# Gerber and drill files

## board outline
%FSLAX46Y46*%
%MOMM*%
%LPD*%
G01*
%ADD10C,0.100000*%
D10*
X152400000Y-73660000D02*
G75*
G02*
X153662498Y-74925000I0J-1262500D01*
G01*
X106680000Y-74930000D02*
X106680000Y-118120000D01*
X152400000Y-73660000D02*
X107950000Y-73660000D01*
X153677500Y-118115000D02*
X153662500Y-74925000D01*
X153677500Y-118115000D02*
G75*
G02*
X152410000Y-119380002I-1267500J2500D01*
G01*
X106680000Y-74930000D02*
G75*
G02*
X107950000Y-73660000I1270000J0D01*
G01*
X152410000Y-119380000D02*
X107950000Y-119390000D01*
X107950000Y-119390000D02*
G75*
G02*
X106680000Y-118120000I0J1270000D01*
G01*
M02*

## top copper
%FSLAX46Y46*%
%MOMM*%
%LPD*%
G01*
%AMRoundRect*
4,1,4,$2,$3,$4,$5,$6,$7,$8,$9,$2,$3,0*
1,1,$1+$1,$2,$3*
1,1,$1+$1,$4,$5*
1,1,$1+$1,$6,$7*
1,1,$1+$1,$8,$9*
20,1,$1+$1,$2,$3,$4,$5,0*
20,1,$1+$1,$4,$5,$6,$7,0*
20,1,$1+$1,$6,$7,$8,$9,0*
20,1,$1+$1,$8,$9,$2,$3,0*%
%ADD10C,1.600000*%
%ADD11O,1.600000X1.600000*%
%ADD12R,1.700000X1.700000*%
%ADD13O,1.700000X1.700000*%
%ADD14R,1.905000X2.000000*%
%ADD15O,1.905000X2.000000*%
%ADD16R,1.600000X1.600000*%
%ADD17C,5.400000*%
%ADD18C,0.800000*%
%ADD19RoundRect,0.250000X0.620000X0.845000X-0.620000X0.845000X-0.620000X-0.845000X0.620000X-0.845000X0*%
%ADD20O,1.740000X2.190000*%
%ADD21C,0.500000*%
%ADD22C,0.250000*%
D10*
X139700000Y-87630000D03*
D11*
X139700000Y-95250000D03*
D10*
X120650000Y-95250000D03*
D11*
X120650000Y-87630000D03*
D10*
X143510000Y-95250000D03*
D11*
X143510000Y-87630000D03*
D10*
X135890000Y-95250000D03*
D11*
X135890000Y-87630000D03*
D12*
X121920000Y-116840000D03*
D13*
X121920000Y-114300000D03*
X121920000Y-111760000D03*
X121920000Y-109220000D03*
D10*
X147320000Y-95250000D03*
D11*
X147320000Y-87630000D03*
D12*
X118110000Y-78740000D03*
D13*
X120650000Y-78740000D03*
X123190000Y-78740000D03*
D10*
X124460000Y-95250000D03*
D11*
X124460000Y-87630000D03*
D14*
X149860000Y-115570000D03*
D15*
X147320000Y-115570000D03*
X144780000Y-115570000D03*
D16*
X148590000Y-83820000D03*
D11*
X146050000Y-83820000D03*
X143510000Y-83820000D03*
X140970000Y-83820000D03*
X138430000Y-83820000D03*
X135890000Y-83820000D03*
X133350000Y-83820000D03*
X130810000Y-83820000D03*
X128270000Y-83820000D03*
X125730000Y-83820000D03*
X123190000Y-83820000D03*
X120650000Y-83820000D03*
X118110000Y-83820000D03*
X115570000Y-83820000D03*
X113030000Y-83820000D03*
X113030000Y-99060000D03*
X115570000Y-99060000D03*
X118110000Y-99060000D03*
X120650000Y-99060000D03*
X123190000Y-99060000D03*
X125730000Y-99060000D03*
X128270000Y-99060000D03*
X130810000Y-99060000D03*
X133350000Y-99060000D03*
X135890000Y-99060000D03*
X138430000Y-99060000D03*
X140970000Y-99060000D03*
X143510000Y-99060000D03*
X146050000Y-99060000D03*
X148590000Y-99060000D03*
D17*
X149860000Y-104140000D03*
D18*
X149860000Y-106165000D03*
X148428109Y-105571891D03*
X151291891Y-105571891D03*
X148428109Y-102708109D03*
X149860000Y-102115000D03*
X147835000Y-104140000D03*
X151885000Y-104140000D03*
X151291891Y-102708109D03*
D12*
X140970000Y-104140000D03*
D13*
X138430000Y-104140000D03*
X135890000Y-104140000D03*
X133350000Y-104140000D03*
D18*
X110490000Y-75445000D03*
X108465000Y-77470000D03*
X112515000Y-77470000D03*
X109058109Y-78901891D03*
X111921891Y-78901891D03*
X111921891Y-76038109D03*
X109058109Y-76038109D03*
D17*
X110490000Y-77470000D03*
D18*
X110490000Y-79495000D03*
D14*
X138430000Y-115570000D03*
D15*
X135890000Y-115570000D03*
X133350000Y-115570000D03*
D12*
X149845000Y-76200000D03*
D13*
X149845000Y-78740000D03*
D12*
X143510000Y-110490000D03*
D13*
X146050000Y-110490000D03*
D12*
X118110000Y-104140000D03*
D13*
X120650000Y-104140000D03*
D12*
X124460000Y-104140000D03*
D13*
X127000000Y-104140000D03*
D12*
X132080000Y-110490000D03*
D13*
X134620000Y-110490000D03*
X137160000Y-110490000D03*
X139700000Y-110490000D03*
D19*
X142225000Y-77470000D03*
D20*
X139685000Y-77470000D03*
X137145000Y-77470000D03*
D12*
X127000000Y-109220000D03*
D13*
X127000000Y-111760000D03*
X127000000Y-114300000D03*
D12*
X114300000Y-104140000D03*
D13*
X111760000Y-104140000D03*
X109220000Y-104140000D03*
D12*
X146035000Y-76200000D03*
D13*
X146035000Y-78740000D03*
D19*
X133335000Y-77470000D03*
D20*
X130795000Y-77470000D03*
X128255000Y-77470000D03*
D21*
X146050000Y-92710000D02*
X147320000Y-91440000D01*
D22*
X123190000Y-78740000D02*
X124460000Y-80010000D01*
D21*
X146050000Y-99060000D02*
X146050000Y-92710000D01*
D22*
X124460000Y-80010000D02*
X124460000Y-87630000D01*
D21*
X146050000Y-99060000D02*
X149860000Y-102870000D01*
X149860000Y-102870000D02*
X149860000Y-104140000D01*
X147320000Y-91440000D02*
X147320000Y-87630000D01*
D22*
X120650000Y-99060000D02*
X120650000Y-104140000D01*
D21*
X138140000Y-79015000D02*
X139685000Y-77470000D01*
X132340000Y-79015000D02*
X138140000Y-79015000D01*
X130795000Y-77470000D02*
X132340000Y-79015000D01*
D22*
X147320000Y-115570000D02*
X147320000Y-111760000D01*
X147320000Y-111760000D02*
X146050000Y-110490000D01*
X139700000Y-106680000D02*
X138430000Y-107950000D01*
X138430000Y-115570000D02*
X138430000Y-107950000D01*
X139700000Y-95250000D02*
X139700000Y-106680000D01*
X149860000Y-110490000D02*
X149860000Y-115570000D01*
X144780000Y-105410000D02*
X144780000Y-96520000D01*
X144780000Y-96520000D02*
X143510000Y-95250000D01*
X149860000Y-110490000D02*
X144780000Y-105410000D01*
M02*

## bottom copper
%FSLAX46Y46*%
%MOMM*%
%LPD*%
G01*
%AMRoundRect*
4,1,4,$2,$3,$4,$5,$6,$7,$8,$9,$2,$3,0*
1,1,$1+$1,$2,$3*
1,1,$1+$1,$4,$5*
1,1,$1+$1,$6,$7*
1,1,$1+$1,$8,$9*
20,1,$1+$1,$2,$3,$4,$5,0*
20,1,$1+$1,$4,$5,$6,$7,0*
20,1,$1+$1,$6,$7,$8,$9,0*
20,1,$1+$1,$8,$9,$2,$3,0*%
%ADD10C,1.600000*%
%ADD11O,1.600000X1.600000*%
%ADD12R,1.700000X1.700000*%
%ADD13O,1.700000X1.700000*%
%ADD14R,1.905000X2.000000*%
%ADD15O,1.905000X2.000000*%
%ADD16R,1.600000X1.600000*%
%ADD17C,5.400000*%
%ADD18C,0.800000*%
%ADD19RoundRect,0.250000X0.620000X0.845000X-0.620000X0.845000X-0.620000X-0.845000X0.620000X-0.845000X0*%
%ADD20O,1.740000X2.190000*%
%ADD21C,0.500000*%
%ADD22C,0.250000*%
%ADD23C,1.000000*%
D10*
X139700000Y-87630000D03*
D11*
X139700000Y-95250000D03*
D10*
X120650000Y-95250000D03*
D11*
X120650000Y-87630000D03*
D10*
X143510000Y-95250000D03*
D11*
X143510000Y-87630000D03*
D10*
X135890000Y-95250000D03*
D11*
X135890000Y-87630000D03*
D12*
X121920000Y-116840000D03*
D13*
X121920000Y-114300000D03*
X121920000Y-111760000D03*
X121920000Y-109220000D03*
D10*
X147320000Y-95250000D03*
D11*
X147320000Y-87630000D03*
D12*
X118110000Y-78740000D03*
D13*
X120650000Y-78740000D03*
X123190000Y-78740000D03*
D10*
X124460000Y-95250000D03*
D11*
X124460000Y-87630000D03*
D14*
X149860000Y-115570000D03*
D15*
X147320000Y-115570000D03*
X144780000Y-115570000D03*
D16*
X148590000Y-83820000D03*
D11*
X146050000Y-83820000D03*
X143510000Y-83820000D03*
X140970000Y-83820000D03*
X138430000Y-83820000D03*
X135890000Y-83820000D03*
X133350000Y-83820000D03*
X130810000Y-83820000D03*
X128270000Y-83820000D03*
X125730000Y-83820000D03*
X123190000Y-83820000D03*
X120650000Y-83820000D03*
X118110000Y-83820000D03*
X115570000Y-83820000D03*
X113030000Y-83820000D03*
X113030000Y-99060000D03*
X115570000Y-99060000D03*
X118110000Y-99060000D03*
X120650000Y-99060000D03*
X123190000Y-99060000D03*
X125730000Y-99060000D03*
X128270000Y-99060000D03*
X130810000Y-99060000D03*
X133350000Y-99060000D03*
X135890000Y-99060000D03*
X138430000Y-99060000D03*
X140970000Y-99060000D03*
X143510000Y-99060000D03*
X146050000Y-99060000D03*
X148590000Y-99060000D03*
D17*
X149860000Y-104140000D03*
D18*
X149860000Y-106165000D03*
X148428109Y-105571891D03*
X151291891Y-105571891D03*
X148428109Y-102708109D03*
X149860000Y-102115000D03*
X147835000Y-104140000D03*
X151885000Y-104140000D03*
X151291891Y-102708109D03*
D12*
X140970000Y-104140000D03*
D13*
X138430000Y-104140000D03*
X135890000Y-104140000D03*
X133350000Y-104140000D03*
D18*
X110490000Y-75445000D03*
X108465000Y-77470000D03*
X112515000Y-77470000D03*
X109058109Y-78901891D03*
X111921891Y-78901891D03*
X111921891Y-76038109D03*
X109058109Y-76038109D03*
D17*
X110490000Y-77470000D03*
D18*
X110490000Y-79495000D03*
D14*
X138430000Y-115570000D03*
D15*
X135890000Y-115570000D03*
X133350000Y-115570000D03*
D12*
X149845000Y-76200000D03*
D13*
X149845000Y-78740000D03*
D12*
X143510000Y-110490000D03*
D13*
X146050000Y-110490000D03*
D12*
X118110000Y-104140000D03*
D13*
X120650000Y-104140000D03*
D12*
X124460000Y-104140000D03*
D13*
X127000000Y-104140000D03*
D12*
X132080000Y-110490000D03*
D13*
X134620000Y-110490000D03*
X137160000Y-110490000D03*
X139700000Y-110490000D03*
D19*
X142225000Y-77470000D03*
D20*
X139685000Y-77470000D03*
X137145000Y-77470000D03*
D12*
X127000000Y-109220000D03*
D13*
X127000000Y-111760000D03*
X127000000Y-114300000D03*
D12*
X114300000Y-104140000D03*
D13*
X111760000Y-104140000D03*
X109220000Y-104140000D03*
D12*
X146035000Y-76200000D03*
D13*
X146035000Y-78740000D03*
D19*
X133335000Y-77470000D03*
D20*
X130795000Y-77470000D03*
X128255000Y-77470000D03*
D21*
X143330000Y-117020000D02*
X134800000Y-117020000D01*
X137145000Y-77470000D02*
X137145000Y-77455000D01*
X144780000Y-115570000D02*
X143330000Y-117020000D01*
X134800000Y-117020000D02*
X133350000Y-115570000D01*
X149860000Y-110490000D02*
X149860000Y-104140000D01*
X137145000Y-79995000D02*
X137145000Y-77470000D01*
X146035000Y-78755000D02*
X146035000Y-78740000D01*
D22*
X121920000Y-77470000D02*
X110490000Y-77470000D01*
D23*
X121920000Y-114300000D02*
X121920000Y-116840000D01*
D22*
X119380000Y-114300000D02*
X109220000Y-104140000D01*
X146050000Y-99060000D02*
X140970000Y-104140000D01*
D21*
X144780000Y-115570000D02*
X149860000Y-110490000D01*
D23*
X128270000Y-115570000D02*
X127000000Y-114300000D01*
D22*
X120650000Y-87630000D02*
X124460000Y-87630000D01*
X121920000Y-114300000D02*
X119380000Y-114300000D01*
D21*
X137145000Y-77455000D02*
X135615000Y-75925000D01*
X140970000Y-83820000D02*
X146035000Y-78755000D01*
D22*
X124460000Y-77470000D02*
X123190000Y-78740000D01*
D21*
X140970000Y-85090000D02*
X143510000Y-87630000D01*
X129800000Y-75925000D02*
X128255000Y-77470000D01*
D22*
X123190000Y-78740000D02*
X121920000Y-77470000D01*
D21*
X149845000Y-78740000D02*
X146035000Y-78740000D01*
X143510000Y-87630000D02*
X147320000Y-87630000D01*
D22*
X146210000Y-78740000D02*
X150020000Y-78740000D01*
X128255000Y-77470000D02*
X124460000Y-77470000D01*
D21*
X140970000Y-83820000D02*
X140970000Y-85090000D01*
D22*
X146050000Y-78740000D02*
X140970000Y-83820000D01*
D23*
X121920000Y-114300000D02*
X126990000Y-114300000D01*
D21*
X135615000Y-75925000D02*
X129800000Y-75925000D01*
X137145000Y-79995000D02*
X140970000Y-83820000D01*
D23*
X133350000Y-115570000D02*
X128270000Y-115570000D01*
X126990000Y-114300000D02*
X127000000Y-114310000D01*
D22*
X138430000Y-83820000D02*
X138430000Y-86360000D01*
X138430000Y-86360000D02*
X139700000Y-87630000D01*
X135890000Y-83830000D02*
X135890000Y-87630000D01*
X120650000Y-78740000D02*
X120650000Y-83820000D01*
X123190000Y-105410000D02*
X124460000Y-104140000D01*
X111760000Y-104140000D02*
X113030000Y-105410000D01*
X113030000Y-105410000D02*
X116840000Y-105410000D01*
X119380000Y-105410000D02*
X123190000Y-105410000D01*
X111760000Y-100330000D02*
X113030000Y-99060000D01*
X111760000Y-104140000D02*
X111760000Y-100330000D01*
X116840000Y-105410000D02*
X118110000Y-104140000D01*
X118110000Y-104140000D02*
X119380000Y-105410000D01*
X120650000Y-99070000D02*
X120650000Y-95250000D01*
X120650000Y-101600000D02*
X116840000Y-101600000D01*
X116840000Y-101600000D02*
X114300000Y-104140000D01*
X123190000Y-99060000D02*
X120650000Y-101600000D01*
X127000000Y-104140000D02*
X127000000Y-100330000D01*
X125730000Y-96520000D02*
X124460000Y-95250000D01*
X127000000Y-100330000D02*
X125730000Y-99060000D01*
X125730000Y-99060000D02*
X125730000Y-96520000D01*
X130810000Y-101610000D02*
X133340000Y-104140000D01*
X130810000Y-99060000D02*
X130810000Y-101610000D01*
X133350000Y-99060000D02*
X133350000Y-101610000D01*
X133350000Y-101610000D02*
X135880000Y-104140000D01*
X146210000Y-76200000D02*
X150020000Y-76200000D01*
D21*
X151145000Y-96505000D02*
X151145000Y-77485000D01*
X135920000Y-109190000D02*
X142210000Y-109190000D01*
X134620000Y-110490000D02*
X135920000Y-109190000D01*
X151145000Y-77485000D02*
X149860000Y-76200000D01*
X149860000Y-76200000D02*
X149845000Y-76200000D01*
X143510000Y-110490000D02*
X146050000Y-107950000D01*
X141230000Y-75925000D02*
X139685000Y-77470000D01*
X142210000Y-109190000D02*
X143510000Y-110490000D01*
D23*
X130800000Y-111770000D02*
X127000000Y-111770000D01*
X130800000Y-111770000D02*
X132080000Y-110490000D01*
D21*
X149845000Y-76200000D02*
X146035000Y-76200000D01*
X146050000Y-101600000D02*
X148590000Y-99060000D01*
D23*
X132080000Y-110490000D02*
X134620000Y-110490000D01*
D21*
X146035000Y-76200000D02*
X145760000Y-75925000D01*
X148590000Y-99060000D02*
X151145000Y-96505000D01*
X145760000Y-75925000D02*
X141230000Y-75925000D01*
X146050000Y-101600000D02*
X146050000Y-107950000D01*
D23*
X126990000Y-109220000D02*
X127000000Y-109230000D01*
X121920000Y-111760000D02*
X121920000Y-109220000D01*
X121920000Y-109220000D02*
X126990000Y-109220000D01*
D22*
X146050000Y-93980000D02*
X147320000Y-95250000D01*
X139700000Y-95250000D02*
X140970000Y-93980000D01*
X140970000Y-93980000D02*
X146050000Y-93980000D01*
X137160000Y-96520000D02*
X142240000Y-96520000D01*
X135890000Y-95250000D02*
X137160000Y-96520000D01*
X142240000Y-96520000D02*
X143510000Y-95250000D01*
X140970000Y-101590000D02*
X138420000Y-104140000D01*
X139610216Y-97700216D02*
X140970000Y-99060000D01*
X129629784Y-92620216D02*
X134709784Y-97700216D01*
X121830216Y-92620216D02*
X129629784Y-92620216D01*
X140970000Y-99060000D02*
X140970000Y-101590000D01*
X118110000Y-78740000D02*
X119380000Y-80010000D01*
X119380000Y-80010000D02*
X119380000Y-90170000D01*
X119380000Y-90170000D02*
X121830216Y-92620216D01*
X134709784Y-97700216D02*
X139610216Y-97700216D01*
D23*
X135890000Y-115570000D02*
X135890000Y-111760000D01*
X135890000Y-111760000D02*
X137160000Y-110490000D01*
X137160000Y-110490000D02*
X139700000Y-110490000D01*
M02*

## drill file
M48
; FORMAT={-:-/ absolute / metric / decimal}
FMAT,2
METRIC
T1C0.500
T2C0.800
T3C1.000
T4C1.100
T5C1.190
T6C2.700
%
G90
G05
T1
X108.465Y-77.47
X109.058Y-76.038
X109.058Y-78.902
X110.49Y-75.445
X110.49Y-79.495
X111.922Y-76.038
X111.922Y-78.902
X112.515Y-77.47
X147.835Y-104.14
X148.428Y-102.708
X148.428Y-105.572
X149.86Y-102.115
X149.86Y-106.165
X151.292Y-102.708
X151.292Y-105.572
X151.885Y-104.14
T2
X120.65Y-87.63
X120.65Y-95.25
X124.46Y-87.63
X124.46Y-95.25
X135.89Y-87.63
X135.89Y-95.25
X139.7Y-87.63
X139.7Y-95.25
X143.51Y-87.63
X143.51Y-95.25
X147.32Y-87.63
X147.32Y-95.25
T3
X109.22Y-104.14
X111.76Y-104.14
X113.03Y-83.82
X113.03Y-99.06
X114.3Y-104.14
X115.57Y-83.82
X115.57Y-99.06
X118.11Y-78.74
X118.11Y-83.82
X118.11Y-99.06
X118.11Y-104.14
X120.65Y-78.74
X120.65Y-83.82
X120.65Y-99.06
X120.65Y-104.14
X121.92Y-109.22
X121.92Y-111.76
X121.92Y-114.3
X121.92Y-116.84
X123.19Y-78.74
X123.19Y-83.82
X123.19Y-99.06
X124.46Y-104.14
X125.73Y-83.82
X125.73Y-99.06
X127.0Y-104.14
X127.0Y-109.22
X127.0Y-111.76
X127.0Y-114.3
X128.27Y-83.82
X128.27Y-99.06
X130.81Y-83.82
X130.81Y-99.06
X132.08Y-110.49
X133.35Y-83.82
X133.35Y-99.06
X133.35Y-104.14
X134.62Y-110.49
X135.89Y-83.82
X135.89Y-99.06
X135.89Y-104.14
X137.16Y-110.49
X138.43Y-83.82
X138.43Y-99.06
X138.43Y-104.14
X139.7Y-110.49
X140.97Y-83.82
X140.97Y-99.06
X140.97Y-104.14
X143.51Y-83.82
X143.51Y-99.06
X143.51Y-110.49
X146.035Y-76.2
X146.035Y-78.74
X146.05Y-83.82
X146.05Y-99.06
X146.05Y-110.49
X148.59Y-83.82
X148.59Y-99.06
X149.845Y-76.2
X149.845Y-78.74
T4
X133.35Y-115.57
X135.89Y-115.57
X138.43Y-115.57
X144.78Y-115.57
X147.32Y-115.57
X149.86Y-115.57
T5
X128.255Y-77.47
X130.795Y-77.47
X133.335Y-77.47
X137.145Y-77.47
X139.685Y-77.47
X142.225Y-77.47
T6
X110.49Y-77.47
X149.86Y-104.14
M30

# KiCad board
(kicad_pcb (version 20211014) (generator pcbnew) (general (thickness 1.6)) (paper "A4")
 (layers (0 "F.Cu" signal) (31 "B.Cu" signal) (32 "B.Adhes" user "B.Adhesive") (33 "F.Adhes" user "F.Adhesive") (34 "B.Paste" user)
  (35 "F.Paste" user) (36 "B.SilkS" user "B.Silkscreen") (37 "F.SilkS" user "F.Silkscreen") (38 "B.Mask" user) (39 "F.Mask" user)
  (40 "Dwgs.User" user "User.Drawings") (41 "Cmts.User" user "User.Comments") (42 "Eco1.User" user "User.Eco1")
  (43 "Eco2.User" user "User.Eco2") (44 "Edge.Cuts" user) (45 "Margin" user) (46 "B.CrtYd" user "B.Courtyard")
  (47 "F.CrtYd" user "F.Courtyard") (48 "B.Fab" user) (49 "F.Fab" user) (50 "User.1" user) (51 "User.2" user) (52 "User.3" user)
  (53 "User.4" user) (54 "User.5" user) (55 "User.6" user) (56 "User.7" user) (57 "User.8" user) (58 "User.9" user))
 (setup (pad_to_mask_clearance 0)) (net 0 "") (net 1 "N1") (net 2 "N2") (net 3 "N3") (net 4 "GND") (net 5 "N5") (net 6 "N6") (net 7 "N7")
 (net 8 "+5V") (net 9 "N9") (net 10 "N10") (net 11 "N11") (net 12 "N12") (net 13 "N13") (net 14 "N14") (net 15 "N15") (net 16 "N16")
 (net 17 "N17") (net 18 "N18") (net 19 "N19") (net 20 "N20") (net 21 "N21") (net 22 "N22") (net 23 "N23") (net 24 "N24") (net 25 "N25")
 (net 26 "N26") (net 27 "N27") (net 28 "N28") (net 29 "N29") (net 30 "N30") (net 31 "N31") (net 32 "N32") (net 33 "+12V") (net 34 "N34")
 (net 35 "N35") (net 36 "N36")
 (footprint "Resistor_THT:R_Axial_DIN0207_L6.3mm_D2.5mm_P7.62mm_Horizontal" (layer "F.Cu") (at 139.7 87.63 -90)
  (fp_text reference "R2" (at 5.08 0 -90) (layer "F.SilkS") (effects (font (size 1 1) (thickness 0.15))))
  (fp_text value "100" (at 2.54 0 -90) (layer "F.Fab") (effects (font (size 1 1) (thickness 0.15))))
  (pad "1" thru_hole circle (at 0 0 270) (size 1.6 1.6) (drill 0.8) (layers *.Cu *.Mask) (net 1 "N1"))
  (pad "2" thru_hole oval (at 7.62 0 270) (size 1.6 1.6) (drill 0.8) (layers *.Cu *.Mask) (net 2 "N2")))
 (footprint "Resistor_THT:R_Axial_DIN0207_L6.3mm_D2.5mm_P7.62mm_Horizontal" (layer "F.Cu") (at 120.65 95.25 90)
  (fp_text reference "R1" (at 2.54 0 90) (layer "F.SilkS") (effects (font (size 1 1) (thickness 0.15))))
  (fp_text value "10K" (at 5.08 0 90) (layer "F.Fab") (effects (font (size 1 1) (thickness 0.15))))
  (pad "1" thru_hole circle (at 0 0 90) (size 1.6 1.6) (drill 0.8) (layers *.Cu *.Mask) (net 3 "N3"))
  (pad "2" thru_hole oval (at 7.62 0 90) (size 1.6 1.6) (drill 0.8) (layers *.Cu *.Mask) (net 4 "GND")))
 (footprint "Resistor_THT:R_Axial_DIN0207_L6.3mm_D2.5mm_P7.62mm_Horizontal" (layer "F.Cu") (at 143.51 95.25 90)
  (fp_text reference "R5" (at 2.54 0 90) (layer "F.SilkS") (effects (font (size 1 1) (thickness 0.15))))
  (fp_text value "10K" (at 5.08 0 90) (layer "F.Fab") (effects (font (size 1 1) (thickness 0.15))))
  (pad "1" thru_hole circle (at 0 0 90) (size 1.6 1.6) (drill 0.8) (layers *.Cu *.Mask) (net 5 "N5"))
  (pad "2" thru_hole oval (at 7.62 0 90) (size 1.6 1.6) (drill 0.8) (layers *.Cu *.Mask) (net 4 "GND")))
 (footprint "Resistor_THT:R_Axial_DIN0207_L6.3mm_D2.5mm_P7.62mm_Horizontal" (layer "F.Cu") (at 135.89 95.25 90)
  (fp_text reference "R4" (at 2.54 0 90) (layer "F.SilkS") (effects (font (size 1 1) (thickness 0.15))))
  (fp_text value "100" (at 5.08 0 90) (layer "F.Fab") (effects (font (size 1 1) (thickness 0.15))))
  (pad "1" thru_hole circle (at 0 0 90) (size 1.6 1.6) (drill 0.8) (layers *.Cu *.Mask) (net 5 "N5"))
  (pad "2" thru_hole oval (at 7.62 0 90) (size 1.6 1.6) (drill 0.8) (layers *.Cu *.Mask) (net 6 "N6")))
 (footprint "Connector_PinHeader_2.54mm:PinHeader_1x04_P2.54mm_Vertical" (layer "F.Cu") (at 121.92 116.84 180)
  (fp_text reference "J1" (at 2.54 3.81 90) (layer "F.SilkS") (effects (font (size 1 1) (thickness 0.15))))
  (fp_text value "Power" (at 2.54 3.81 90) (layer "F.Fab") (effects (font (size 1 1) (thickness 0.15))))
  (pad "1" thru_hole rect (at 0 0 180) (size 1.7 1.7) (drill 1) (layers *.Cu *.Mask) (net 4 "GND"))
  (pad "2" thru_hole oval (at 0 2.54 180) (size 1.7 1.7) (drill 1) (layers *.Cu *.Mask) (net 4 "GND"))
  (pad "3" thru_hole oval (at 0 5.08 180) (size 1.7 1.7) (drill 1) (layers *.Cu *.Mask) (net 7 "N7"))
  (pad "4" thru_hole oval (at 0 7.62 180) (size 1.7 1.7) (drill 1) (layers *.Cu *.Mask) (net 7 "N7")))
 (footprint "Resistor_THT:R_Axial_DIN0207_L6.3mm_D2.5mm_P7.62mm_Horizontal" (layer "F.Cu") (at 147.32 95.25 90)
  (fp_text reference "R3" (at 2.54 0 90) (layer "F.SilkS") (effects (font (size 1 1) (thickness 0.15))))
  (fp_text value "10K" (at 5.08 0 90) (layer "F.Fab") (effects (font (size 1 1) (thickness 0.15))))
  (pad "1" thru_hole circle (at 0 0 90) (size 1.6 1.6) (drill 0.8) (layers *.Cu *.Mask) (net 2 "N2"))
  (pad "2" thru_hole oval (at 7.62 0 90) (size 1.6 1.6) (drill 0.8) (layers *.Cu *.Mask) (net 4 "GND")))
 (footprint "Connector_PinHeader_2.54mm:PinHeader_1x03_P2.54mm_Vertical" (layer "F.Cu") (at 118.11 78.74 90)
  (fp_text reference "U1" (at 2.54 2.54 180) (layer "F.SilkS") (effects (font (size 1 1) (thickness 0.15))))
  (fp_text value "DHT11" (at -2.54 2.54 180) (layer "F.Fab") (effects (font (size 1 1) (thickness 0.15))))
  (pad "1" thru_hole rect (at 0 0 90) (size 1.7 1.7) (drill 1) (layers *.Cu *.Mask) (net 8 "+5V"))
  (pad "2" thru_hole oval (at 0 2.54 90) (size 1.7 1.7) (drill 1) (layers *.Cu *.Mask) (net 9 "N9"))
  (pad "3" thru_hole oval (at 0 5.08 90) (size 1.7 1.7) (drill 1) (layers *.Cu *.Mask) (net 4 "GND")))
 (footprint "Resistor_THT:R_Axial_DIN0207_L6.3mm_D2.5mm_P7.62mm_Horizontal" (layer "F.Cu") (at 124.46 95.25 90)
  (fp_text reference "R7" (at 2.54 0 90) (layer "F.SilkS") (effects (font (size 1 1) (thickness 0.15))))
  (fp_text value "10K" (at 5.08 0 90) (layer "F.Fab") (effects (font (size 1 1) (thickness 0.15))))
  (pad "1" thru_hole circle (at 0 0 90) (size 1.6 1.6) (drill 0.8) (layers *.Cu *.Mask) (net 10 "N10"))
  (pad "2" thru_hole oval (at 7.62 0 90) (size 1.6 1.6) (drill 0.8) (layers *.Cu *.Mask) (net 4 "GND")))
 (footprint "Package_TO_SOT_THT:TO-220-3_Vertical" (layer "F.Cu") (at 149.86 115.57 180)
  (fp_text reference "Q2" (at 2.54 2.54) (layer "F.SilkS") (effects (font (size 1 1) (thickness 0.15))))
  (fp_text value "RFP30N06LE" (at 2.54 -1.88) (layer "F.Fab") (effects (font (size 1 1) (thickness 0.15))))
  (pad "1" thru_hole rect (at 0 0 180) (size 1.905 2) (drill 1.1) (layers *.Cu *.Mask) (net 5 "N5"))
  (pad "2" thru_hole oval (at 2.54 0 180) (size 1.905 2) (drill 1.1) (layers *.Cu *.Mask) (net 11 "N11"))
  (pad "3" thru_hole oval (at 5.08 0 180) (size 1.905 2) (drill 1.1) (layers *.Cu *.Mask) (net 4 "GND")))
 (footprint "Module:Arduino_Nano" (layer "F.Cu") (at 148.59 83.82 -90)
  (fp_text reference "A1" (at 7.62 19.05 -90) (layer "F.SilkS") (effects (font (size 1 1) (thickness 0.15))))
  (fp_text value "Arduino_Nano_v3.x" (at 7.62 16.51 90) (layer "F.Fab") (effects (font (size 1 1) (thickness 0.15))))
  (pad "1" thru_hole rect (at 0 0 270) (size 1.6 1.6) (drill 1) (layers *.Cu *.Mask) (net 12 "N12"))
  (pad "2" thru_hole oval (at 0 2.54 270) (size 1.6 1.6) (drill 1) (layers *.Cu *.Mask) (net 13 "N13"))
  (pad "3" thru_hole oval (at 0 5.08 270) (size 1.6 1.6) (drill 1) (layers *.Cu *.Mask) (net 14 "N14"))
  (pad "4" thru_hole oval (at 0 7.62 270) (size 1.6 1.6) (drill 1) (layers *.Cu *.Mask) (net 4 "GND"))
  (pad "5" thru_hole oval (at 0 10.16 270) (size 1.6 1.6) (drill 1) (layers *.Cu *.Mask) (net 1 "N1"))
  (pad "6" thru_hole oval (at 0 12.7 270) (size 1.6 1.6) (drill 1) (layers *.Cu *.Mask) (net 6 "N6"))
  (pad "7" thru_hole oval (at 0 15.24 270) (size 1.6 1.6) (drill 1) (layers *.Cu *.Mask) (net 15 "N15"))
  (pad "8" thru_hole oval (at 0 17.78 270) (size 1.6 1.6) (drill 1) (layers *.Cu *.Mask) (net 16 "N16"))
  (pad "9" thru_hole oval (at 0 20.32 270) (size 1.6 1.6) (drill 1) (layers *.Cu *.Mask) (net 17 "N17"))
  (pad "10" thru_hole oval (at 0 22.86 270) (size 1.6 1.6) (drill 1) (layers *.Cu *.Mask) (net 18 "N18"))
  (pad "11" thru_hole oval (at 0 25.4 270) (size 1.6 1.6) (drill 1) (layers *.Cu *.Mask) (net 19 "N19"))
  (pad "12" thru_hole oval (at 0 27.94 270) (size 1.6 1.6) (drill 1) (layers *.Cu *.Mask) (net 9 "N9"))
  (pad "13" thru_hole oval (at 0 30.48 270) (size 1.6 1.6) (drill 1) (layers *.Cu *.Mask) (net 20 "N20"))
  (pad "14" thru_hole oval (at 0 33.02 270) (size 1.6 1.6) (drill 1) (layers *.Cu *.Mask) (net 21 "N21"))
  (pad "15" thru_hole oval (at 0 35.56 270) (size 1.6 1.6) (drill 1) (layers *.Cu *.Mask) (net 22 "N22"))
  (pad "16" thru_hole oval (at 15.24 35.56 270) (size 1.6 1.6) (drill 1) (layers *.Cu *.Mask) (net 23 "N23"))
  (pad "17" thru_hole oval (at 15.24 33.02 270) (size 1.6 1.6) (drill 1) (layers *.Cu *.Mask) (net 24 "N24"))
  (pad "18" thru_hole oval (at 15.24 30.48 270) (size 1.6 1.6) (drill 1) (layers *.Cu *.Mask) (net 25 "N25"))
  (pad "19" thru_hole oval (at 15.24 27.94 270) (size 1.6 1.6) (drill 1) (layers *.Cu *.Mask) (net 3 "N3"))
  (pad "20" thru_hole oval (at 15.24 25.4 270) (size 1.6 1.6) (drill 1) (layers *.Cu *.Mask) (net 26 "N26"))
  (pad "21" thru_hole oval (at 15.24 22.86 270) (size 1.6 1.6) (drill 1) (layers *.Cu *.Mask) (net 10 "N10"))
  (pad "22" thru_hole oval (at 15.24 20.32 270) (size 1.6 1.6) (drill 1) (layers *.Cu *.Mask) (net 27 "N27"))
  (pad "23" thru_hole oval (at 15.24 17.78 270) (size 1.6 1.6) (drill 1) (layers *.Cu *.Mask) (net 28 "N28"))
  (pad "24" thru_hole oval (at 15.24 15.24 270) (size 1.6 1.6) (drill 1) (layers *.Cu *.Mask) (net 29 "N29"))
  (pad "25" thru_hole oval (at 15.24 12.7 270) (size 1.6 1.6) (drill 1) (layers *.Cu *.Mask) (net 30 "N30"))
  (pad "26" thru_hole oval (at 15.24 10.16 270) (size 1.6 1.6) (drill 1) (layers *.Cu *.Mask) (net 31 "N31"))
  (pad "27" thru_hole oval (at 15.24 7.62 270) (size 1.6 1.6) (drill 1) (layers *.Cu *.Mask) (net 8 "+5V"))
  (pad "28" thru_hole oval (at 15.24 5.08 270) (size 1.6 1.6) (drill 1) (layers *.Cu *.Mask) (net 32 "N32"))
  (pad "29" thru_hole oval (at 15.24 2.54 270) (size 1.6 1.6) (drill 1) (layers *.Cu *.Mask) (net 4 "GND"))
  (pad "30" thru_hole oval (at 15.24 0 270) (size 1.6 1.6) (drill 1) (layers *.Cu *.Mask) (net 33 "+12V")))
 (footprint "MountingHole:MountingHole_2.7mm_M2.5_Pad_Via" (layer "F.Cu") (at 149.86 104.14)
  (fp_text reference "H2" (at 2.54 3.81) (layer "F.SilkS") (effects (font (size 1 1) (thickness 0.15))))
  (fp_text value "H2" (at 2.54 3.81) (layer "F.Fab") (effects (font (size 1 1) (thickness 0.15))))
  (pad "1" thru_hole circle (at 0 0) (size 5.4 5.4) (drill 2.7) (layers *.Cu *.Mask) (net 4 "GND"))
  (pad "1" thru_hole circle (at 0 2.025) (size 0.8 0.8) (drill 0.5) (layers *.Cu *.Mask) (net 4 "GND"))
  (pad "1" thru_hole circle (at -1.431891 1.431891) (size 0.8 0.8) (drill 0.5) (layers *.Cu *.Mask) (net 4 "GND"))
  (pad "1" thru_hole circle (at 1.431891 1.431891) (size 0.8 0.8) (drill 0.5) (layers *.Cu *.Mask) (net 4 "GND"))
  (pad "1" thru_hole circle (at -1.431891 -1.431891) (size 0.8 0.8) (drill 0.5) (layers *.Cu *.Mask) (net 4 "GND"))
  (pad "1" thru_hole circle (at 0 -2.025) (size 0.8 0.8) (drill 0.5) (layers *.Cu *.Mask) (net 4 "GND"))
  (pad "1" thru_hole circle (at -2.025 0) (size 0.8 0.8) (drill 0.5) (layers *.Cu *.Mask) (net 4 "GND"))
  (pad "1" thru_hole circle (at 2.025 0) (size 0.8 0.8) (drill 0.5) (layers *.Cu *.Mask) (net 4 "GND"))
  (pad "1" thru_hole circle (at 1.431891 -1.431891) (size 0.8 0.8) (drill 0.5) (layers *.Cu *.Mask) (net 4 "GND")))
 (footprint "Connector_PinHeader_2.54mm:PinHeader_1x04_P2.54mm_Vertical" (layer "F.Cu") (at 140.97 104.14 -90)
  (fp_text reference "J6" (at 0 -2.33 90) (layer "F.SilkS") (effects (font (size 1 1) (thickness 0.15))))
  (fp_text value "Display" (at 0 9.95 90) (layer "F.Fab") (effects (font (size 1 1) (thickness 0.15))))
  (pad "1" thru_hole rect (at 0 0 270) (size 1.7 1.7) (drill 1) (layers *.Cu *.Mask) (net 4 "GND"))
  (pad "2" thru_hole oval (at 0 2.54 270) (size 1.7 1.7) (drill 1) (layers *.Cu *.Mask) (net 8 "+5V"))
  (pad "3" thru_hole oval (at 0 5.08 270) (size 1.7 1.7) (drill 1) (layers *.Cu *.Mask) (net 29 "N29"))
  (pad "4" thru_hole oval (at 0 7.62 270) (size 1.7 1.7) (drill 1) (layers *.Cu *.Mask) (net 28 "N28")))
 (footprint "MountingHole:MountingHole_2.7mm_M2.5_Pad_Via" (layer "F.Cu") (at 110.49 77.47)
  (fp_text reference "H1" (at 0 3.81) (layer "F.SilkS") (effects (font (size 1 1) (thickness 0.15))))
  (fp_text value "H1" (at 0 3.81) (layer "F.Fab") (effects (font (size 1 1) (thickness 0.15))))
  (pad "1" thru_hole circle (at 0 -2.025) (size 0.8 0.8) (drill 0.5) (layers *.Cu *.Mask) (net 4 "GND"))
  (pad "1" thru_hole circle (at -2.025 0) (size 0.8 0.8) (drill 0.5) (layers *.Cu *.Mask) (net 4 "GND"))
  (pad "1" thru_hole circle (at 2.025 0) (size 0.8 0.8) (drill 0.5) (layers *.Cu *.Mask) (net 4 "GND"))
  (pad "1" thru_hole circle (at -1.431891 1.431891) (size 0.8 0.8) (drill 0.5) (layers *.Cu *.Mask) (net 4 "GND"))
  (pad "1" thru_hole circle (at 1.431891 1.431891) (size 0.8 0.8) (drill 0.5) (layers *.Cu *.Mask) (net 4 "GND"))
  (pad "1" thru_hole circle (at 1.431891 -1.431891) (size 0.8 0.8) (drill 0.5) (layers *.Cu *.Mask) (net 4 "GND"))
  (pad "1" thru_hole circle (at -1.431891 -1.431891) (size 0.8 0.8) (drill 0.5) (layers *.Cu *.Mask) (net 4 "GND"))
  (pad "1" thru_hole circle (at 0 0) (size 5.4 5.4) (drill 2.7) (layers *.Cu *.Mask) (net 4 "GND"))
  (pad "1" thru_hole circle (at 0 2.025) (size 0.8 0.8) (drill 0.5) (layers *.Cu *.Mask) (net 4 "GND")))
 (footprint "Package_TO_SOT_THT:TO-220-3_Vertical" (layer "F.Cu") (at 138.43 115.57 180)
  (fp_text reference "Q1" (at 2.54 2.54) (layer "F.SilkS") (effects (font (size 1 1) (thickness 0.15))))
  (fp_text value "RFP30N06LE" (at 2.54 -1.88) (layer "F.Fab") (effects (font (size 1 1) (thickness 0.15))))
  (pad "1" thru_hole rect (at 0 0 180) (size 1.905 2) (drill 1.1) (layers *.Cu *.Mask) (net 2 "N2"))
  (pad "2" thru_hole oval (at 2.54 0 180) (size 1.905 2) (drill 1.1) (layers *.Cu *.Mask) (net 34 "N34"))
  (pad "3" thru_hole oval (at 5.08 0 180) (size 1.905 2) (drill 1.1) (layers *.Cu *.Mask) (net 4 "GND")))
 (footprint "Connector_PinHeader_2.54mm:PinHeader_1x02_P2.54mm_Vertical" (layer "B.Cu") (at 149.845 76.2 180)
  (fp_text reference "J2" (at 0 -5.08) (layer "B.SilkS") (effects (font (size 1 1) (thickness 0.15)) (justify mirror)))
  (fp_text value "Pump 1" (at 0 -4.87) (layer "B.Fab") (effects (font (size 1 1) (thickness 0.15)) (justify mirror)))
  (pad "1" thru_hole rect (at 0 0 180) (size 1.7 1.7) (drill 1) (layers *.Cu *.Mask) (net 33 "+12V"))
  (pad "2" thru_hole oval (at 0 -2.54 180) (size 1.7 1.7) (drill 1) (layers *.Cu *.Mask) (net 4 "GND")))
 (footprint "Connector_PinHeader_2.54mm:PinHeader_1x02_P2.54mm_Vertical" (layer "B.Cu") (at 143.51 110.49 -90)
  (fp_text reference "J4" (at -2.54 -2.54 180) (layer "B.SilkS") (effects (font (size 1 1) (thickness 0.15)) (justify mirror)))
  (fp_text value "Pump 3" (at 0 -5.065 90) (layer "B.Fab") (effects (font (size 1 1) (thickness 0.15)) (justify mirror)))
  (pad "1" thru_hole rect (at 0 0 270) (size 1.7 1.7) (drill 1) (layers *.Cu *.Mask) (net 33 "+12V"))
  (pad "2" thru_hole oval (at 0 -2.54 270) (size 1.7 1.7) (drill 1) (layers *.Cu *.Mask) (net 11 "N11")))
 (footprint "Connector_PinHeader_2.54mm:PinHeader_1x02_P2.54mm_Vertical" (layer "B.Cu") (at 118.11 104.14 -90)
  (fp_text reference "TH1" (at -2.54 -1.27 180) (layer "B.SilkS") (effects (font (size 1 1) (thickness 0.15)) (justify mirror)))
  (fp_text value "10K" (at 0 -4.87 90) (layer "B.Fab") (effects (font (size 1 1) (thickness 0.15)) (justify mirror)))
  (pad "1" thru_hole rect (at 0 0 270) (size 1.7 1.7) (drill 1) (layers *.Cu *.Mask) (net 23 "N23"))
  (pad "2" thru_hole oval (at 0 -2.54 270) (size 1.7 1.7) (drill 1) (layers *.Cu *.Mask) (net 3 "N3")))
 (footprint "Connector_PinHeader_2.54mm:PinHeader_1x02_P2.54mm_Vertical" (layer "B.Cu") (at 124.46 104.14 -90)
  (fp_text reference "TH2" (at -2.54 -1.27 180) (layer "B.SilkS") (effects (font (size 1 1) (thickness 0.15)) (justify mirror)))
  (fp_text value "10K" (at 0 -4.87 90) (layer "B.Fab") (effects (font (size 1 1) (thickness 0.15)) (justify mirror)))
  (pad "1" thru_hole rect (at 0 0 270) (size 1.7 1.7) (drill 1) (layers *.Cu *.Mask) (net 23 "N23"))
  (pad "2" thru_hole oval (at 0 -2.54 270) (size 1.7 1.7) (drill 1) (layers *.Cu *.Mask) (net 10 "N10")))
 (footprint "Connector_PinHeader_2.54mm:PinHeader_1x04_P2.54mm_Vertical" (layer "B.Cu") (at 132.08 110.49 -90)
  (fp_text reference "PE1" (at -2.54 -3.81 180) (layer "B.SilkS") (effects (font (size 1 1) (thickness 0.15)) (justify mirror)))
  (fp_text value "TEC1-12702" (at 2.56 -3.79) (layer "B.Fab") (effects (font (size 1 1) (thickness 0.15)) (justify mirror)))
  (pad "1" thru_hole rect (at 0 0 270) (size 1.7 1.7) (drill 1) (layers *.Cu *.Mask) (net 33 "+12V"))
  (pad "2" thru_hole oval (at 0 -2.54 270) (size 1.7 1.7) (drill 1) (layers *.Cu *.Mask) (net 33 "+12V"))
  (pad "3" thru_hole oval (at 0 -5.08 270) (size 1.7 1.7) (drill 1) (layers *.Cu *.Mask) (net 34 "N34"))
  (pad "4" thru_hole oval (at 0 -7.62 270) (size 1.7 1.7) (drill 1) (layers *.Cu *.Mask) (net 34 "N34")))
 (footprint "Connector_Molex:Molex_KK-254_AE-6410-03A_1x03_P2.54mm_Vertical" (layer "B.Cu") (at 142.225 77.47 180)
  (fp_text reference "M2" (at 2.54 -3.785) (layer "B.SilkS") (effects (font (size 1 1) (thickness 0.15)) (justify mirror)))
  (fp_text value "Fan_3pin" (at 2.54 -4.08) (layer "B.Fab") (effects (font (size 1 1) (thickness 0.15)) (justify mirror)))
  (pad "1" thru_hole roundrect (at 0 0 180) (size 1.74 2.19) (drill 1.19) (layers *.Cu *.Mask) (roundrect_rratio 0.1436781609)
   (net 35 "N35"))
  (pad "2" thru_hole oval (at 2.54 0 180) (size 1.74 2.19) (drill 1.19) (layers *.Cu *.Mask) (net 33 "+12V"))
  (pad "3" thru_hole oval (at 5.08 0 180) (size 1.74 2.19) (drill 1.19) (layers *.Cu *.Mask) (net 4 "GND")))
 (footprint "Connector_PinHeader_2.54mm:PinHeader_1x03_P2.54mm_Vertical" (layer "B.Cu") (at 127 109.22 180)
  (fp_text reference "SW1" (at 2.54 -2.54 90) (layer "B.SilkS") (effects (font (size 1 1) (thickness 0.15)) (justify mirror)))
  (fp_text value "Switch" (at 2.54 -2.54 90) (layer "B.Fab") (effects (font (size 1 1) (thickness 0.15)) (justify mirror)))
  (pad "1" thru_hole rect (at 0 0 180) (size 1.7 1.7) (drill 1) (layers *.Cu *.Mask) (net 7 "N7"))
  (pad "2" thru_hole oval (at 0 -2.54 180) (size 1.7 1.7) (drill 1) (layers *.Cu *.Mask) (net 33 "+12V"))
  (pad "3" thru_hole oval (at 0 -5.08 180) (size 1.7 1.7) (drill 1) (layers *.Cu *.Mask) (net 4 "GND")))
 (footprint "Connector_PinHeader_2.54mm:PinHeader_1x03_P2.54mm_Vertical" (layer "B.Cu") (at 114.3 104.14 90)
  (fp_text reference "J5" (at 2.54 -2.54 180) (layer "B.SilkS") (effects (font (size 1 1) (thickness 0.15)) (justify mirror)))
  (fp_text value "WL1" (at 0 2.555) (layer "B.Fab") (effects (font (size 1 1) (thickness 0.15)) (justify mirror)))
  (pad "1" thru_hole rect (at 0 0 90) (size 1.7 1.7) (drill 1) (layers *.Cu *.Mask) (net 26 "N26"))
  (pad "2" thru_hole oval (at 0 -2.54 90) (size 1.7 1.7) (drill 1) (layers *.Cu *.Mask) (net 23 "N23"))
  (pad "3" thru_hole oval (at 0 -5.08 90) (size 1.7 1.7) (drill 1) (layers *.Cu *.Mask) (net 4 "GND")))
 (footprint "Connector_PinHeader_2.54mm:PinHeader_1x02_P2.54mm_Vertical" (layer "B.Cu") (at 146.035 76.2 180)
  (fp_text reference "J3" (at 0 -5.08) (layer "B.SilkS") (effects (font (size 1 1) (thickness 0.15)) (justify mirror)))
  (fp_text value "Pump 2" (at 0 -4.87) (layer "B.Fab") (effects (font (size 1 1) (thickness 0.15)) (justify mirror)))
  (pad "1" thru_hole rect (at 0 0 180) (size 1.7 1.7) (drill 1) (layers *.Cu *.Mask) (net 33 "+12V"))
  (pad "2" thru_hole oval (at 0 -2.54 180) (size 1.7 1.7) (drill 1) (layers *.Cu *.Mask) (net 4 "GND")))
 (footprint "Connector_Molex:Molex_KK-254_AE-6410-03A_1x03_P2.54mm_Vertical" (layer "B.Cu") (at 133.335 77.47 180)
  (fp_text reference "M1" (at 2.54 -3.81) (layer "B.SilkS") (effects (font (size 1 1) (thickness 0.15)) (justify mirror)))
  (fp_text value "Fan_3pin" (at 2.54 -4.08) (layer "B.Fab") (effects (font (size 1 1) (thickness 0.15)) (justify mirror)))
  (pad "1" thru_hole roundrect (at 0 0 180) (size 1.74 2.19) (drill 1.19) (layers *.Cu *.Mask) (roundrect_rratio 0.1436781609)
   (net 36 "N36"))
  (pad "2" thru_hole oval (at 2.54 0 180) (size 1.74 2.19) (drill 1.19) (layers *.Cu *.Mask) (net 33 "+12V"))
  (pad "3" thru_hole oval (at 5.08 0 180) (size 1.74 2.19) (drill 1.19) (layers *.Cu *.Mask) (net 4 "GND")))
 (gr_arc (start 152.4 73.66) (mid 153.293606 74.030662) (end 153.6625 74.925) (layer "Edge.Cuts") (width 0.1))
 (gr_line (start 106.68 74.93) (end 106.68 118.12) (layer "Edge.Cuts") (width 0.1))
 (gr_line (start 152.4 73.66) (end 107.95 73.66) (layer "Edge.Cuts") (width 0.1))
 (gr_line (start 153.6775 118.115) (end 153.6625 74.925) (layer "Edge.Cuts") (width 0.1))
 (gr_arc (start 153.6775 118.115) (mid 153.305374 119.009641) (end 152.41 119.38) (layer "Edge.Cuts") (width 0.1))
 (gr_arc (start 106.68 74.93) (mid 107.051974 74.031974) (end 107.95 73.66) (layer "Edge.Cuts") (width 0.1))
 (gr_line (start 152.41 119.38) (end 107.95 119.39) (layer "Edge.Cuts") (width 0.1))
 (gr_arc (start 107.95 119.39) (mid 107.051974 119.018026) (end 106.68 118.12) (layer "Edge.Cuts") (width 0.1))
 (segment (start 146.05 92.71) (end 147.32 91.44) (width 0.5) (layer "F.Cu") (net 4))
 (segment (start 123.19 78.74) (end 124.46 80.01) (width 0.25) (layer "F.Cu") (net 4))
 (segment (start 146.05 99.06) (end 146.05 92.71) (width 0.5) (layer "F.Cu") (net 4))
 (segment (start 124.46 80.01) (end 124.46 87.63) (width 0.25) (layer "F.Cu") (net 4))
 (segment (start 146.05 99.06) (end 149.86 102.87) (width 0.5) (layer "F.Cu") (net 4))
 (segment (start 149.86 102.87) (end 149.86 104.14) (width 0.5) (layer "F.Cu") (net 4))
 (segment (start 147.32 91.44) (end 147.32 87.63) (width 0.5) (layer "F.Cu") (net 4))
 (segment (start 143.33 117.02) (end 134.8 117.02) (width 0.5) (layer "B.Cu") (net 4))
 (segment (start 137.145 77.47) (end 137.145 77.455) (width 0.5) (layer "B.Cu") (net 4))
 (segment (start 144.78 115.57) (end 143.33 117.02) (width 0.5) (layer "B.Cu") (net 4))
 (segment (start 134.8 117.02) (end 133.35 115.57) (width 0.5) (layer "B.Cu") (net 4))
 (segment (start 149.86 110.49) (end 149.86 104.14) (width 0.5) (layer "B.Cu") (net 4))
 (segment (start 137.145 79.995) (end 137.145 77.47) (width 0.5) (layer "B.Cu") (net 4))
 (segment (start 146.035 78.755) (end 146.035 78.74) (width 0.5) (layer "B.Cu") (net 4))
 (segment (start 121.92 77.47) (end 110.49 77.47) (width 0.25) (layer "B.Cu") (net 4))
 (segment (start 121.92 114.3) (end 121.92 116.84) (width 1) (layer "B.Cu") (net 4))
 (segment (start 119.38 114.3) (end 109.22 104.14) (width 0.25) (layer "B.Cu") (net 4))
 (segment (start 146.05 99.06) (end 140.97 104.14) (width 0.25) (layer "B.Cu") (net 4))
 (segment (start 144.78 115.57) (end 149.86 110.49) (width 0.5) (layer "B.Cu") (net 4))
 (segment (start 128.27 115.57) (end 127 114.3) (width 1) (layer "B.Cu") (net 4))
 (segment (start 120.65 87.63) (end 124.46 87.63) (width 0.25) (layer "B.Cu") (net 4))
 (segment (start 121.92 114.3) (end 119.38 114.3) (width 0.25) (layer "B.Cu") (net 4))
 (segment (start 137.145 77.455) (end 135.615 75.925) (width 0.5) (layer "B.Cu") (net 4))
 (segment (start 140.97 83.82) (end 146.035 78.755) (width 0.5) (layer "B.Cu") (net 4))
 (segment (start 124.46 77.47) (end 123.19 78.74) (width 0.25) (layer "B.Cu") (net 4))
 (segment (start 140.97 85.09) (end 143.51 87.63) (width 0.5) (layer "B.Cu") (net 4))
 (segment (start 129.8 75.925) (end 128.255 77.47) (width 0.5) (layer "B.Cu") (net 4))
 (segment (start 123.19 78.74) (end 121.92 77.47) (width 0.25) (layer "B.Cu") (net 4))
 (segment (start 149.845 78.74) (end 146.035 78.74) (width 0.5) (layer "B.Cu") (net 4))
 (segment (start 143.51 87.63) (end 147.32 87.63) (width 0.5) (layer "B.Cu") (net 4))
 (segment (start 146.21 78.74) (end 150.02 78.74) (width 0.25) (layer "B.Cu") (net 4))
 (segment (start 128.255 77.47) (end 124.46 77.47) (width 0.25) (layer "B.Cu") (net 4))
 (segment (start 140.97 83.82) (end 140.97 85.09) (width 0.5) (layer "B.Cu") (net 4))
 (segment (start 146.05 78.74) (end 140.97 83.82) (width 0.25) (layer "B.Cu") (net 4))
 (segment (start 121.92 114.3) (end 126.99 114.3) (width 1) (layer "B.Cu") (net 4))
 (segment (start 135.615 75.925) (end 129.8 75.925) (width 0.5) (layer "B.Cu") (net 4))
 (segment (start 137.145 79.995) (end 140.97 83.82) (width 0.5) (layer "B.Cu") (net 4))
 (segment (start 133.35 115.57) (end 128.27 115.57) (width 1) (layer "B.Cu") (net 4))
 (segment (start 126.99 114.3) (end 127 114.31) (width 1) (layer "B.Cu") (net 4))
 (segment (start 138.43 83.82) (end 138.43 86.36) (width 0.25) (layer "B.Cu") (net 1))
 (segment (start 138.43 86.36) (end 139.7 87.63) (width 0.25) (layer "B.Cu") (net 1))
 (segment (start 135.89 83.83) (end 135.89 87.63) (width 0.25) (layer "B.Cu") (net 6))
 (segment (start 120.65 78.74) (end 120.65 83.82) (width 0.25) (layer "B.Cu") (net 9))
 (segment (start 123.19 105.41) (end 124.46 104.14) (width 0.25) (layer "B.Cu") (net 23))
 (segment (start 111.76 104.14) (end 113.03 105.41) (width 0.25) (layer "B.Cu") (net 23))
 (segment (start 113.03 105.41) (end 116.84 105.41) (width 0.25) (layer "B.Cu") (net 23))
 (segment (start 119.38 105.41) (end 123.19 105.41) (width 0.25) (layer "B.Cu") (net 23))
 (segment (start 111.76 100.33) (end 113.03 99.06) (width 0.25) (layer "B.Cu") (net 23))
 (segment (start 111.76 104.14) (end 111.76 100.33) (width 0.25) (layer "B.Cu") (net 23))
 (segment (start 116.84 105.41) (end 118.11 104.14) (width 0.25) (layer "B.Cu") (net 23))
 (segment (start 118.11 104.14) (end 119.38 105.41) (width 0.25) (layer "B.Cu") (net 23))
 (segment (start 120.65 99.06) (end 120.65 104.14) (width 0.25) (layer "F.Cu") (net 3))
 (segment (start 120.65 99.07) (end 120.65 95.25) (width 0.25) (layer "B.Cu") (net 3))
 (segment (start 120.65 101.6) (end 116.84 101.6) (width 0.25) (layer "B.Cu") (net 26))
 (segment (start 116.84 101.6) (end 114.3 104.14) (width 0.25) (layer "B.Cu") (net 26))
 (segment (start 123.19 99.06) (end 120.65 101.6) (width 0.25) (layer "B.Cu") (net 26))
 (segment (start 127 104.14) (end 127 100.33) (width 0.25) (layer "B.Cu") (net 10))
 (segment (start 125.73 96.52) (end 124.46 95.25) (width 0.25) (layer "B.Cu") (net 10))
 (segment (start 127 100.33) (end 125.73 99.06) (width 0.25) (layer "B.Cu") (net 10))
 (segment (start 125.73 99.06) (end 125.73 96.52) (width 0.25) (layer "B.Cu") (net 10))
 (segment (start 130.81 101.61) (end 133.34 104.14) (width 0.25) (layer "B.Cu") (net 28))
 (segment (start 130.81 99.06) (end 130.81 101.61) (width 0.25) (layer "B.Cu") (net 28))
 (segment (start 133.35 99.06) (end 133.35 101.61) (width 0.25) (layer "B.Cu") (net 29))
 (segment (start 133.35 101.61) (end 135.88 104.14) (width 0.25) (layer "B.Cu") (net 29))
 (segment (start 138.14 79.015) (end 139.685 77.47) (width 0.5) (layer "F.Cu") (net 33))
 (segment (start 132.34 79.015) (end 138.14 79.015) (width 0.5) (layer "F.Cu") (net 33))
 (segment (start 130.795 77.47) (end 132.34 79.015) (width 0.5) (layer "F.Cu") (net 33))
 (segment (start 146.21 76.2) (end 150.02 76.2) (width 0.25) (layer "B.Cu") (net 33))
 (segment (start 151.145 96.505) (end 151.145 77.485) (width 0.5) (layer "B.Cu") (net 33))
 (segment (start 135.92 109.19) (end 142.21 109.19) (width 0.5) (layer "B.Cu") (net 33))
 (segment (start 134.62 110.49) (end 135.92 109.19) (width 0.5) (layer "B.Cu") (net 33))
 (segment (start 151.145 77.485) (end 149.86 76.2) (width 0.5) (layer "B.Cu") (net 33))
 (segment (start 149.86 76.2) (end 149.845 76.2) (width 0.5) (layer "B.Cu") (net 33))
 (segment (start 143.51 110.49) (end 146.05 107.95) (width 0.5) (layer "B.Cu") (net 33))
 (segment (start 141.23 75.925) (end 139.685 77.47) (width 0.5) (layer "B.Cu") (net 33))
 (segment (start 142.21 109.19) (end 143.51 110.49) (width 0.5) (layer "B.Cu") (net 33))
 (segment (start 130.8 111.77) (end 127 111.77) (width 1) (layer "B.Cu") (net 33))
 (segment (start 130.8 111.77) (end 132.08 110.49) (width 1) (layer "B.Cu") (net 33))
 (segment (start 149.845 76.2) (end 146.035 76.2) (width 0.5) (layer "B.Cu") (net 33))
 (segment (start 146.05 101.6) (end 148.59 99.06) (width 0.5) (layer "B.Cu") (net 33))
 (segment (start 132.08 110.49) (end 134.62 110.49) (width 1) (layer "B.Cu") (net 33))
 (segment (start 146.035 76.2) (end 145.76 75.925) (width 0.5) (layer "B.Cu") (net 33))
 (segment (start 148.59 99.06) (end 151.145 96.505) (width 0.5) (layer "B.Cu") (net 33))
 (segment (start 145.76 75.925) (end 141.23 75.925) (width 0.5) (layer "B.Cu") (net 33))
 (segment (start 146.05 101.6) (end 146.05 107.95) (width 0.5) (layer "B.Cu") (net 33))
 (segment (start 126.99 109.22) (end 127 109.23) (width 1) (layer "B.Cu") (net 7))
 (segment (start 121.92 111.76) (end 121.92 109.22) (width 1) (layer "B.Cu") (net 7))
 (segment (start 121.92 109.22) (end 126.99 109.22) (width 1) (layer "B.Cu") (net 7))
 (segment (start 147.32 115.57) (end 147.32 111.76) (width 0.25) (layer "F.Cu") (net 11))
 (segment (start 147.32 111.76) (end 146.05 110.49) (width 0.25) (layer "F.Cu") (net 11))
 (segment (start 139.7 106.68) (end 138.43 107.95) (width 0.25) (layer "F.Cu") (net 2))
 (segment (start 138.43 115.57) (end 138.43 107.95) (width 0.25) (layer "F.Cu") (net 2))
 (segment (start 139.7 95.25) (end 139.7 106.68) (width 0.25) (layer "F.Cu") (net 2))
 (segment (start 146.05 93.98) (end 147.32 95.25) (width 0.25) (layer "B.Cu") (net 2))
 (segment (start 139.7 95.25) (end 140.97 93.98) (width 0.25) (layer "B.Cu") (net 2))
 (segment (start 140.97 93.98) (end 146.05 93.98) (width 0.25) (layer "B.Cu") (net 2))
 (segment (start 149.86 110.49) (end 149.86 115.57) (width 0.25) (layer "F.Cu") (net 5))
 (segment (start 144.78 105.41) (end 144.78 96.52) (width 0.25) (layer "F.Cu") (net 5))
 (segment (start 144.78 96.52) (end 143.51 95.25) (width 0.25) (layer "F.Cu") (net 5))
 (segment (start 149.86 110.49) (end 144.78 105.41) (width 0.25) (layer "F.Cu") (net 5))
 (segment (start 137.16 96.52) (end 142.24 96.52) (width 0.25) (layer "B.Cu") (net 5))
 (segment (start 135.89 95.25) (end 137.16 96.52) (width 0.25) (layer "B.Cu") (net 5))
 (segment (start 142.24 96.52) (end 143.51 95.25) (width 0.25) (layer "B.Cu") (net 5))
 (segment (start 140.97 101.59) (end 138.42 104.14) (width 0.25) (layer "B.Cu") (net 8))
 (segment (start 139.610216 97.700216) (end 140.97 99.06) (width 0.25) (layer "B.Cu") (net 8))
 (segment (start 129.629784 92.620216) (end 134.709784 97.700216) (width 0.25) (layer "B.Cu") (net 8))
 (segment (start 121.830216 92.620216) (end 129.629784 92.620216) (width 0.25) (layer "B.Cu") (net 8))
 (segment (start 140.97 99.06) (end 140.97 101.59) (width 0.25) (layer "B.Cu") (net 8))
 (segment (start 118.11 78.74) (end 119.38 80.01) (width 0.25) (layer "B.Cu") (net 8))
 (segment (start 119.38 80.01) (end 119.38 90.17) (width 0.25) (layer "B.Cu") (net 8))
 (segment (start 119.38 90.17) (end 121.830216 92.620216) (width 0.25) (layer "B.Cu") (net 8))
 (segment (start 134.709784 97.700216) (end 139.610216 97.700216) (width 0.25) (layer "B.Cu") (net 8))
 (segment (start 135.89 115.57) (end 135.89 111.76) (width 1) (layer "B.Cu") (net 34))
 (segment (start 135.89 111.76) (end 137.16 110.49) (width 1) (layer "B.Cu") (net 34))
 (segment (start 137.16 110.49) (end 139.7 110.49) (width 1) (layer "B.Cu") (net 34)))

